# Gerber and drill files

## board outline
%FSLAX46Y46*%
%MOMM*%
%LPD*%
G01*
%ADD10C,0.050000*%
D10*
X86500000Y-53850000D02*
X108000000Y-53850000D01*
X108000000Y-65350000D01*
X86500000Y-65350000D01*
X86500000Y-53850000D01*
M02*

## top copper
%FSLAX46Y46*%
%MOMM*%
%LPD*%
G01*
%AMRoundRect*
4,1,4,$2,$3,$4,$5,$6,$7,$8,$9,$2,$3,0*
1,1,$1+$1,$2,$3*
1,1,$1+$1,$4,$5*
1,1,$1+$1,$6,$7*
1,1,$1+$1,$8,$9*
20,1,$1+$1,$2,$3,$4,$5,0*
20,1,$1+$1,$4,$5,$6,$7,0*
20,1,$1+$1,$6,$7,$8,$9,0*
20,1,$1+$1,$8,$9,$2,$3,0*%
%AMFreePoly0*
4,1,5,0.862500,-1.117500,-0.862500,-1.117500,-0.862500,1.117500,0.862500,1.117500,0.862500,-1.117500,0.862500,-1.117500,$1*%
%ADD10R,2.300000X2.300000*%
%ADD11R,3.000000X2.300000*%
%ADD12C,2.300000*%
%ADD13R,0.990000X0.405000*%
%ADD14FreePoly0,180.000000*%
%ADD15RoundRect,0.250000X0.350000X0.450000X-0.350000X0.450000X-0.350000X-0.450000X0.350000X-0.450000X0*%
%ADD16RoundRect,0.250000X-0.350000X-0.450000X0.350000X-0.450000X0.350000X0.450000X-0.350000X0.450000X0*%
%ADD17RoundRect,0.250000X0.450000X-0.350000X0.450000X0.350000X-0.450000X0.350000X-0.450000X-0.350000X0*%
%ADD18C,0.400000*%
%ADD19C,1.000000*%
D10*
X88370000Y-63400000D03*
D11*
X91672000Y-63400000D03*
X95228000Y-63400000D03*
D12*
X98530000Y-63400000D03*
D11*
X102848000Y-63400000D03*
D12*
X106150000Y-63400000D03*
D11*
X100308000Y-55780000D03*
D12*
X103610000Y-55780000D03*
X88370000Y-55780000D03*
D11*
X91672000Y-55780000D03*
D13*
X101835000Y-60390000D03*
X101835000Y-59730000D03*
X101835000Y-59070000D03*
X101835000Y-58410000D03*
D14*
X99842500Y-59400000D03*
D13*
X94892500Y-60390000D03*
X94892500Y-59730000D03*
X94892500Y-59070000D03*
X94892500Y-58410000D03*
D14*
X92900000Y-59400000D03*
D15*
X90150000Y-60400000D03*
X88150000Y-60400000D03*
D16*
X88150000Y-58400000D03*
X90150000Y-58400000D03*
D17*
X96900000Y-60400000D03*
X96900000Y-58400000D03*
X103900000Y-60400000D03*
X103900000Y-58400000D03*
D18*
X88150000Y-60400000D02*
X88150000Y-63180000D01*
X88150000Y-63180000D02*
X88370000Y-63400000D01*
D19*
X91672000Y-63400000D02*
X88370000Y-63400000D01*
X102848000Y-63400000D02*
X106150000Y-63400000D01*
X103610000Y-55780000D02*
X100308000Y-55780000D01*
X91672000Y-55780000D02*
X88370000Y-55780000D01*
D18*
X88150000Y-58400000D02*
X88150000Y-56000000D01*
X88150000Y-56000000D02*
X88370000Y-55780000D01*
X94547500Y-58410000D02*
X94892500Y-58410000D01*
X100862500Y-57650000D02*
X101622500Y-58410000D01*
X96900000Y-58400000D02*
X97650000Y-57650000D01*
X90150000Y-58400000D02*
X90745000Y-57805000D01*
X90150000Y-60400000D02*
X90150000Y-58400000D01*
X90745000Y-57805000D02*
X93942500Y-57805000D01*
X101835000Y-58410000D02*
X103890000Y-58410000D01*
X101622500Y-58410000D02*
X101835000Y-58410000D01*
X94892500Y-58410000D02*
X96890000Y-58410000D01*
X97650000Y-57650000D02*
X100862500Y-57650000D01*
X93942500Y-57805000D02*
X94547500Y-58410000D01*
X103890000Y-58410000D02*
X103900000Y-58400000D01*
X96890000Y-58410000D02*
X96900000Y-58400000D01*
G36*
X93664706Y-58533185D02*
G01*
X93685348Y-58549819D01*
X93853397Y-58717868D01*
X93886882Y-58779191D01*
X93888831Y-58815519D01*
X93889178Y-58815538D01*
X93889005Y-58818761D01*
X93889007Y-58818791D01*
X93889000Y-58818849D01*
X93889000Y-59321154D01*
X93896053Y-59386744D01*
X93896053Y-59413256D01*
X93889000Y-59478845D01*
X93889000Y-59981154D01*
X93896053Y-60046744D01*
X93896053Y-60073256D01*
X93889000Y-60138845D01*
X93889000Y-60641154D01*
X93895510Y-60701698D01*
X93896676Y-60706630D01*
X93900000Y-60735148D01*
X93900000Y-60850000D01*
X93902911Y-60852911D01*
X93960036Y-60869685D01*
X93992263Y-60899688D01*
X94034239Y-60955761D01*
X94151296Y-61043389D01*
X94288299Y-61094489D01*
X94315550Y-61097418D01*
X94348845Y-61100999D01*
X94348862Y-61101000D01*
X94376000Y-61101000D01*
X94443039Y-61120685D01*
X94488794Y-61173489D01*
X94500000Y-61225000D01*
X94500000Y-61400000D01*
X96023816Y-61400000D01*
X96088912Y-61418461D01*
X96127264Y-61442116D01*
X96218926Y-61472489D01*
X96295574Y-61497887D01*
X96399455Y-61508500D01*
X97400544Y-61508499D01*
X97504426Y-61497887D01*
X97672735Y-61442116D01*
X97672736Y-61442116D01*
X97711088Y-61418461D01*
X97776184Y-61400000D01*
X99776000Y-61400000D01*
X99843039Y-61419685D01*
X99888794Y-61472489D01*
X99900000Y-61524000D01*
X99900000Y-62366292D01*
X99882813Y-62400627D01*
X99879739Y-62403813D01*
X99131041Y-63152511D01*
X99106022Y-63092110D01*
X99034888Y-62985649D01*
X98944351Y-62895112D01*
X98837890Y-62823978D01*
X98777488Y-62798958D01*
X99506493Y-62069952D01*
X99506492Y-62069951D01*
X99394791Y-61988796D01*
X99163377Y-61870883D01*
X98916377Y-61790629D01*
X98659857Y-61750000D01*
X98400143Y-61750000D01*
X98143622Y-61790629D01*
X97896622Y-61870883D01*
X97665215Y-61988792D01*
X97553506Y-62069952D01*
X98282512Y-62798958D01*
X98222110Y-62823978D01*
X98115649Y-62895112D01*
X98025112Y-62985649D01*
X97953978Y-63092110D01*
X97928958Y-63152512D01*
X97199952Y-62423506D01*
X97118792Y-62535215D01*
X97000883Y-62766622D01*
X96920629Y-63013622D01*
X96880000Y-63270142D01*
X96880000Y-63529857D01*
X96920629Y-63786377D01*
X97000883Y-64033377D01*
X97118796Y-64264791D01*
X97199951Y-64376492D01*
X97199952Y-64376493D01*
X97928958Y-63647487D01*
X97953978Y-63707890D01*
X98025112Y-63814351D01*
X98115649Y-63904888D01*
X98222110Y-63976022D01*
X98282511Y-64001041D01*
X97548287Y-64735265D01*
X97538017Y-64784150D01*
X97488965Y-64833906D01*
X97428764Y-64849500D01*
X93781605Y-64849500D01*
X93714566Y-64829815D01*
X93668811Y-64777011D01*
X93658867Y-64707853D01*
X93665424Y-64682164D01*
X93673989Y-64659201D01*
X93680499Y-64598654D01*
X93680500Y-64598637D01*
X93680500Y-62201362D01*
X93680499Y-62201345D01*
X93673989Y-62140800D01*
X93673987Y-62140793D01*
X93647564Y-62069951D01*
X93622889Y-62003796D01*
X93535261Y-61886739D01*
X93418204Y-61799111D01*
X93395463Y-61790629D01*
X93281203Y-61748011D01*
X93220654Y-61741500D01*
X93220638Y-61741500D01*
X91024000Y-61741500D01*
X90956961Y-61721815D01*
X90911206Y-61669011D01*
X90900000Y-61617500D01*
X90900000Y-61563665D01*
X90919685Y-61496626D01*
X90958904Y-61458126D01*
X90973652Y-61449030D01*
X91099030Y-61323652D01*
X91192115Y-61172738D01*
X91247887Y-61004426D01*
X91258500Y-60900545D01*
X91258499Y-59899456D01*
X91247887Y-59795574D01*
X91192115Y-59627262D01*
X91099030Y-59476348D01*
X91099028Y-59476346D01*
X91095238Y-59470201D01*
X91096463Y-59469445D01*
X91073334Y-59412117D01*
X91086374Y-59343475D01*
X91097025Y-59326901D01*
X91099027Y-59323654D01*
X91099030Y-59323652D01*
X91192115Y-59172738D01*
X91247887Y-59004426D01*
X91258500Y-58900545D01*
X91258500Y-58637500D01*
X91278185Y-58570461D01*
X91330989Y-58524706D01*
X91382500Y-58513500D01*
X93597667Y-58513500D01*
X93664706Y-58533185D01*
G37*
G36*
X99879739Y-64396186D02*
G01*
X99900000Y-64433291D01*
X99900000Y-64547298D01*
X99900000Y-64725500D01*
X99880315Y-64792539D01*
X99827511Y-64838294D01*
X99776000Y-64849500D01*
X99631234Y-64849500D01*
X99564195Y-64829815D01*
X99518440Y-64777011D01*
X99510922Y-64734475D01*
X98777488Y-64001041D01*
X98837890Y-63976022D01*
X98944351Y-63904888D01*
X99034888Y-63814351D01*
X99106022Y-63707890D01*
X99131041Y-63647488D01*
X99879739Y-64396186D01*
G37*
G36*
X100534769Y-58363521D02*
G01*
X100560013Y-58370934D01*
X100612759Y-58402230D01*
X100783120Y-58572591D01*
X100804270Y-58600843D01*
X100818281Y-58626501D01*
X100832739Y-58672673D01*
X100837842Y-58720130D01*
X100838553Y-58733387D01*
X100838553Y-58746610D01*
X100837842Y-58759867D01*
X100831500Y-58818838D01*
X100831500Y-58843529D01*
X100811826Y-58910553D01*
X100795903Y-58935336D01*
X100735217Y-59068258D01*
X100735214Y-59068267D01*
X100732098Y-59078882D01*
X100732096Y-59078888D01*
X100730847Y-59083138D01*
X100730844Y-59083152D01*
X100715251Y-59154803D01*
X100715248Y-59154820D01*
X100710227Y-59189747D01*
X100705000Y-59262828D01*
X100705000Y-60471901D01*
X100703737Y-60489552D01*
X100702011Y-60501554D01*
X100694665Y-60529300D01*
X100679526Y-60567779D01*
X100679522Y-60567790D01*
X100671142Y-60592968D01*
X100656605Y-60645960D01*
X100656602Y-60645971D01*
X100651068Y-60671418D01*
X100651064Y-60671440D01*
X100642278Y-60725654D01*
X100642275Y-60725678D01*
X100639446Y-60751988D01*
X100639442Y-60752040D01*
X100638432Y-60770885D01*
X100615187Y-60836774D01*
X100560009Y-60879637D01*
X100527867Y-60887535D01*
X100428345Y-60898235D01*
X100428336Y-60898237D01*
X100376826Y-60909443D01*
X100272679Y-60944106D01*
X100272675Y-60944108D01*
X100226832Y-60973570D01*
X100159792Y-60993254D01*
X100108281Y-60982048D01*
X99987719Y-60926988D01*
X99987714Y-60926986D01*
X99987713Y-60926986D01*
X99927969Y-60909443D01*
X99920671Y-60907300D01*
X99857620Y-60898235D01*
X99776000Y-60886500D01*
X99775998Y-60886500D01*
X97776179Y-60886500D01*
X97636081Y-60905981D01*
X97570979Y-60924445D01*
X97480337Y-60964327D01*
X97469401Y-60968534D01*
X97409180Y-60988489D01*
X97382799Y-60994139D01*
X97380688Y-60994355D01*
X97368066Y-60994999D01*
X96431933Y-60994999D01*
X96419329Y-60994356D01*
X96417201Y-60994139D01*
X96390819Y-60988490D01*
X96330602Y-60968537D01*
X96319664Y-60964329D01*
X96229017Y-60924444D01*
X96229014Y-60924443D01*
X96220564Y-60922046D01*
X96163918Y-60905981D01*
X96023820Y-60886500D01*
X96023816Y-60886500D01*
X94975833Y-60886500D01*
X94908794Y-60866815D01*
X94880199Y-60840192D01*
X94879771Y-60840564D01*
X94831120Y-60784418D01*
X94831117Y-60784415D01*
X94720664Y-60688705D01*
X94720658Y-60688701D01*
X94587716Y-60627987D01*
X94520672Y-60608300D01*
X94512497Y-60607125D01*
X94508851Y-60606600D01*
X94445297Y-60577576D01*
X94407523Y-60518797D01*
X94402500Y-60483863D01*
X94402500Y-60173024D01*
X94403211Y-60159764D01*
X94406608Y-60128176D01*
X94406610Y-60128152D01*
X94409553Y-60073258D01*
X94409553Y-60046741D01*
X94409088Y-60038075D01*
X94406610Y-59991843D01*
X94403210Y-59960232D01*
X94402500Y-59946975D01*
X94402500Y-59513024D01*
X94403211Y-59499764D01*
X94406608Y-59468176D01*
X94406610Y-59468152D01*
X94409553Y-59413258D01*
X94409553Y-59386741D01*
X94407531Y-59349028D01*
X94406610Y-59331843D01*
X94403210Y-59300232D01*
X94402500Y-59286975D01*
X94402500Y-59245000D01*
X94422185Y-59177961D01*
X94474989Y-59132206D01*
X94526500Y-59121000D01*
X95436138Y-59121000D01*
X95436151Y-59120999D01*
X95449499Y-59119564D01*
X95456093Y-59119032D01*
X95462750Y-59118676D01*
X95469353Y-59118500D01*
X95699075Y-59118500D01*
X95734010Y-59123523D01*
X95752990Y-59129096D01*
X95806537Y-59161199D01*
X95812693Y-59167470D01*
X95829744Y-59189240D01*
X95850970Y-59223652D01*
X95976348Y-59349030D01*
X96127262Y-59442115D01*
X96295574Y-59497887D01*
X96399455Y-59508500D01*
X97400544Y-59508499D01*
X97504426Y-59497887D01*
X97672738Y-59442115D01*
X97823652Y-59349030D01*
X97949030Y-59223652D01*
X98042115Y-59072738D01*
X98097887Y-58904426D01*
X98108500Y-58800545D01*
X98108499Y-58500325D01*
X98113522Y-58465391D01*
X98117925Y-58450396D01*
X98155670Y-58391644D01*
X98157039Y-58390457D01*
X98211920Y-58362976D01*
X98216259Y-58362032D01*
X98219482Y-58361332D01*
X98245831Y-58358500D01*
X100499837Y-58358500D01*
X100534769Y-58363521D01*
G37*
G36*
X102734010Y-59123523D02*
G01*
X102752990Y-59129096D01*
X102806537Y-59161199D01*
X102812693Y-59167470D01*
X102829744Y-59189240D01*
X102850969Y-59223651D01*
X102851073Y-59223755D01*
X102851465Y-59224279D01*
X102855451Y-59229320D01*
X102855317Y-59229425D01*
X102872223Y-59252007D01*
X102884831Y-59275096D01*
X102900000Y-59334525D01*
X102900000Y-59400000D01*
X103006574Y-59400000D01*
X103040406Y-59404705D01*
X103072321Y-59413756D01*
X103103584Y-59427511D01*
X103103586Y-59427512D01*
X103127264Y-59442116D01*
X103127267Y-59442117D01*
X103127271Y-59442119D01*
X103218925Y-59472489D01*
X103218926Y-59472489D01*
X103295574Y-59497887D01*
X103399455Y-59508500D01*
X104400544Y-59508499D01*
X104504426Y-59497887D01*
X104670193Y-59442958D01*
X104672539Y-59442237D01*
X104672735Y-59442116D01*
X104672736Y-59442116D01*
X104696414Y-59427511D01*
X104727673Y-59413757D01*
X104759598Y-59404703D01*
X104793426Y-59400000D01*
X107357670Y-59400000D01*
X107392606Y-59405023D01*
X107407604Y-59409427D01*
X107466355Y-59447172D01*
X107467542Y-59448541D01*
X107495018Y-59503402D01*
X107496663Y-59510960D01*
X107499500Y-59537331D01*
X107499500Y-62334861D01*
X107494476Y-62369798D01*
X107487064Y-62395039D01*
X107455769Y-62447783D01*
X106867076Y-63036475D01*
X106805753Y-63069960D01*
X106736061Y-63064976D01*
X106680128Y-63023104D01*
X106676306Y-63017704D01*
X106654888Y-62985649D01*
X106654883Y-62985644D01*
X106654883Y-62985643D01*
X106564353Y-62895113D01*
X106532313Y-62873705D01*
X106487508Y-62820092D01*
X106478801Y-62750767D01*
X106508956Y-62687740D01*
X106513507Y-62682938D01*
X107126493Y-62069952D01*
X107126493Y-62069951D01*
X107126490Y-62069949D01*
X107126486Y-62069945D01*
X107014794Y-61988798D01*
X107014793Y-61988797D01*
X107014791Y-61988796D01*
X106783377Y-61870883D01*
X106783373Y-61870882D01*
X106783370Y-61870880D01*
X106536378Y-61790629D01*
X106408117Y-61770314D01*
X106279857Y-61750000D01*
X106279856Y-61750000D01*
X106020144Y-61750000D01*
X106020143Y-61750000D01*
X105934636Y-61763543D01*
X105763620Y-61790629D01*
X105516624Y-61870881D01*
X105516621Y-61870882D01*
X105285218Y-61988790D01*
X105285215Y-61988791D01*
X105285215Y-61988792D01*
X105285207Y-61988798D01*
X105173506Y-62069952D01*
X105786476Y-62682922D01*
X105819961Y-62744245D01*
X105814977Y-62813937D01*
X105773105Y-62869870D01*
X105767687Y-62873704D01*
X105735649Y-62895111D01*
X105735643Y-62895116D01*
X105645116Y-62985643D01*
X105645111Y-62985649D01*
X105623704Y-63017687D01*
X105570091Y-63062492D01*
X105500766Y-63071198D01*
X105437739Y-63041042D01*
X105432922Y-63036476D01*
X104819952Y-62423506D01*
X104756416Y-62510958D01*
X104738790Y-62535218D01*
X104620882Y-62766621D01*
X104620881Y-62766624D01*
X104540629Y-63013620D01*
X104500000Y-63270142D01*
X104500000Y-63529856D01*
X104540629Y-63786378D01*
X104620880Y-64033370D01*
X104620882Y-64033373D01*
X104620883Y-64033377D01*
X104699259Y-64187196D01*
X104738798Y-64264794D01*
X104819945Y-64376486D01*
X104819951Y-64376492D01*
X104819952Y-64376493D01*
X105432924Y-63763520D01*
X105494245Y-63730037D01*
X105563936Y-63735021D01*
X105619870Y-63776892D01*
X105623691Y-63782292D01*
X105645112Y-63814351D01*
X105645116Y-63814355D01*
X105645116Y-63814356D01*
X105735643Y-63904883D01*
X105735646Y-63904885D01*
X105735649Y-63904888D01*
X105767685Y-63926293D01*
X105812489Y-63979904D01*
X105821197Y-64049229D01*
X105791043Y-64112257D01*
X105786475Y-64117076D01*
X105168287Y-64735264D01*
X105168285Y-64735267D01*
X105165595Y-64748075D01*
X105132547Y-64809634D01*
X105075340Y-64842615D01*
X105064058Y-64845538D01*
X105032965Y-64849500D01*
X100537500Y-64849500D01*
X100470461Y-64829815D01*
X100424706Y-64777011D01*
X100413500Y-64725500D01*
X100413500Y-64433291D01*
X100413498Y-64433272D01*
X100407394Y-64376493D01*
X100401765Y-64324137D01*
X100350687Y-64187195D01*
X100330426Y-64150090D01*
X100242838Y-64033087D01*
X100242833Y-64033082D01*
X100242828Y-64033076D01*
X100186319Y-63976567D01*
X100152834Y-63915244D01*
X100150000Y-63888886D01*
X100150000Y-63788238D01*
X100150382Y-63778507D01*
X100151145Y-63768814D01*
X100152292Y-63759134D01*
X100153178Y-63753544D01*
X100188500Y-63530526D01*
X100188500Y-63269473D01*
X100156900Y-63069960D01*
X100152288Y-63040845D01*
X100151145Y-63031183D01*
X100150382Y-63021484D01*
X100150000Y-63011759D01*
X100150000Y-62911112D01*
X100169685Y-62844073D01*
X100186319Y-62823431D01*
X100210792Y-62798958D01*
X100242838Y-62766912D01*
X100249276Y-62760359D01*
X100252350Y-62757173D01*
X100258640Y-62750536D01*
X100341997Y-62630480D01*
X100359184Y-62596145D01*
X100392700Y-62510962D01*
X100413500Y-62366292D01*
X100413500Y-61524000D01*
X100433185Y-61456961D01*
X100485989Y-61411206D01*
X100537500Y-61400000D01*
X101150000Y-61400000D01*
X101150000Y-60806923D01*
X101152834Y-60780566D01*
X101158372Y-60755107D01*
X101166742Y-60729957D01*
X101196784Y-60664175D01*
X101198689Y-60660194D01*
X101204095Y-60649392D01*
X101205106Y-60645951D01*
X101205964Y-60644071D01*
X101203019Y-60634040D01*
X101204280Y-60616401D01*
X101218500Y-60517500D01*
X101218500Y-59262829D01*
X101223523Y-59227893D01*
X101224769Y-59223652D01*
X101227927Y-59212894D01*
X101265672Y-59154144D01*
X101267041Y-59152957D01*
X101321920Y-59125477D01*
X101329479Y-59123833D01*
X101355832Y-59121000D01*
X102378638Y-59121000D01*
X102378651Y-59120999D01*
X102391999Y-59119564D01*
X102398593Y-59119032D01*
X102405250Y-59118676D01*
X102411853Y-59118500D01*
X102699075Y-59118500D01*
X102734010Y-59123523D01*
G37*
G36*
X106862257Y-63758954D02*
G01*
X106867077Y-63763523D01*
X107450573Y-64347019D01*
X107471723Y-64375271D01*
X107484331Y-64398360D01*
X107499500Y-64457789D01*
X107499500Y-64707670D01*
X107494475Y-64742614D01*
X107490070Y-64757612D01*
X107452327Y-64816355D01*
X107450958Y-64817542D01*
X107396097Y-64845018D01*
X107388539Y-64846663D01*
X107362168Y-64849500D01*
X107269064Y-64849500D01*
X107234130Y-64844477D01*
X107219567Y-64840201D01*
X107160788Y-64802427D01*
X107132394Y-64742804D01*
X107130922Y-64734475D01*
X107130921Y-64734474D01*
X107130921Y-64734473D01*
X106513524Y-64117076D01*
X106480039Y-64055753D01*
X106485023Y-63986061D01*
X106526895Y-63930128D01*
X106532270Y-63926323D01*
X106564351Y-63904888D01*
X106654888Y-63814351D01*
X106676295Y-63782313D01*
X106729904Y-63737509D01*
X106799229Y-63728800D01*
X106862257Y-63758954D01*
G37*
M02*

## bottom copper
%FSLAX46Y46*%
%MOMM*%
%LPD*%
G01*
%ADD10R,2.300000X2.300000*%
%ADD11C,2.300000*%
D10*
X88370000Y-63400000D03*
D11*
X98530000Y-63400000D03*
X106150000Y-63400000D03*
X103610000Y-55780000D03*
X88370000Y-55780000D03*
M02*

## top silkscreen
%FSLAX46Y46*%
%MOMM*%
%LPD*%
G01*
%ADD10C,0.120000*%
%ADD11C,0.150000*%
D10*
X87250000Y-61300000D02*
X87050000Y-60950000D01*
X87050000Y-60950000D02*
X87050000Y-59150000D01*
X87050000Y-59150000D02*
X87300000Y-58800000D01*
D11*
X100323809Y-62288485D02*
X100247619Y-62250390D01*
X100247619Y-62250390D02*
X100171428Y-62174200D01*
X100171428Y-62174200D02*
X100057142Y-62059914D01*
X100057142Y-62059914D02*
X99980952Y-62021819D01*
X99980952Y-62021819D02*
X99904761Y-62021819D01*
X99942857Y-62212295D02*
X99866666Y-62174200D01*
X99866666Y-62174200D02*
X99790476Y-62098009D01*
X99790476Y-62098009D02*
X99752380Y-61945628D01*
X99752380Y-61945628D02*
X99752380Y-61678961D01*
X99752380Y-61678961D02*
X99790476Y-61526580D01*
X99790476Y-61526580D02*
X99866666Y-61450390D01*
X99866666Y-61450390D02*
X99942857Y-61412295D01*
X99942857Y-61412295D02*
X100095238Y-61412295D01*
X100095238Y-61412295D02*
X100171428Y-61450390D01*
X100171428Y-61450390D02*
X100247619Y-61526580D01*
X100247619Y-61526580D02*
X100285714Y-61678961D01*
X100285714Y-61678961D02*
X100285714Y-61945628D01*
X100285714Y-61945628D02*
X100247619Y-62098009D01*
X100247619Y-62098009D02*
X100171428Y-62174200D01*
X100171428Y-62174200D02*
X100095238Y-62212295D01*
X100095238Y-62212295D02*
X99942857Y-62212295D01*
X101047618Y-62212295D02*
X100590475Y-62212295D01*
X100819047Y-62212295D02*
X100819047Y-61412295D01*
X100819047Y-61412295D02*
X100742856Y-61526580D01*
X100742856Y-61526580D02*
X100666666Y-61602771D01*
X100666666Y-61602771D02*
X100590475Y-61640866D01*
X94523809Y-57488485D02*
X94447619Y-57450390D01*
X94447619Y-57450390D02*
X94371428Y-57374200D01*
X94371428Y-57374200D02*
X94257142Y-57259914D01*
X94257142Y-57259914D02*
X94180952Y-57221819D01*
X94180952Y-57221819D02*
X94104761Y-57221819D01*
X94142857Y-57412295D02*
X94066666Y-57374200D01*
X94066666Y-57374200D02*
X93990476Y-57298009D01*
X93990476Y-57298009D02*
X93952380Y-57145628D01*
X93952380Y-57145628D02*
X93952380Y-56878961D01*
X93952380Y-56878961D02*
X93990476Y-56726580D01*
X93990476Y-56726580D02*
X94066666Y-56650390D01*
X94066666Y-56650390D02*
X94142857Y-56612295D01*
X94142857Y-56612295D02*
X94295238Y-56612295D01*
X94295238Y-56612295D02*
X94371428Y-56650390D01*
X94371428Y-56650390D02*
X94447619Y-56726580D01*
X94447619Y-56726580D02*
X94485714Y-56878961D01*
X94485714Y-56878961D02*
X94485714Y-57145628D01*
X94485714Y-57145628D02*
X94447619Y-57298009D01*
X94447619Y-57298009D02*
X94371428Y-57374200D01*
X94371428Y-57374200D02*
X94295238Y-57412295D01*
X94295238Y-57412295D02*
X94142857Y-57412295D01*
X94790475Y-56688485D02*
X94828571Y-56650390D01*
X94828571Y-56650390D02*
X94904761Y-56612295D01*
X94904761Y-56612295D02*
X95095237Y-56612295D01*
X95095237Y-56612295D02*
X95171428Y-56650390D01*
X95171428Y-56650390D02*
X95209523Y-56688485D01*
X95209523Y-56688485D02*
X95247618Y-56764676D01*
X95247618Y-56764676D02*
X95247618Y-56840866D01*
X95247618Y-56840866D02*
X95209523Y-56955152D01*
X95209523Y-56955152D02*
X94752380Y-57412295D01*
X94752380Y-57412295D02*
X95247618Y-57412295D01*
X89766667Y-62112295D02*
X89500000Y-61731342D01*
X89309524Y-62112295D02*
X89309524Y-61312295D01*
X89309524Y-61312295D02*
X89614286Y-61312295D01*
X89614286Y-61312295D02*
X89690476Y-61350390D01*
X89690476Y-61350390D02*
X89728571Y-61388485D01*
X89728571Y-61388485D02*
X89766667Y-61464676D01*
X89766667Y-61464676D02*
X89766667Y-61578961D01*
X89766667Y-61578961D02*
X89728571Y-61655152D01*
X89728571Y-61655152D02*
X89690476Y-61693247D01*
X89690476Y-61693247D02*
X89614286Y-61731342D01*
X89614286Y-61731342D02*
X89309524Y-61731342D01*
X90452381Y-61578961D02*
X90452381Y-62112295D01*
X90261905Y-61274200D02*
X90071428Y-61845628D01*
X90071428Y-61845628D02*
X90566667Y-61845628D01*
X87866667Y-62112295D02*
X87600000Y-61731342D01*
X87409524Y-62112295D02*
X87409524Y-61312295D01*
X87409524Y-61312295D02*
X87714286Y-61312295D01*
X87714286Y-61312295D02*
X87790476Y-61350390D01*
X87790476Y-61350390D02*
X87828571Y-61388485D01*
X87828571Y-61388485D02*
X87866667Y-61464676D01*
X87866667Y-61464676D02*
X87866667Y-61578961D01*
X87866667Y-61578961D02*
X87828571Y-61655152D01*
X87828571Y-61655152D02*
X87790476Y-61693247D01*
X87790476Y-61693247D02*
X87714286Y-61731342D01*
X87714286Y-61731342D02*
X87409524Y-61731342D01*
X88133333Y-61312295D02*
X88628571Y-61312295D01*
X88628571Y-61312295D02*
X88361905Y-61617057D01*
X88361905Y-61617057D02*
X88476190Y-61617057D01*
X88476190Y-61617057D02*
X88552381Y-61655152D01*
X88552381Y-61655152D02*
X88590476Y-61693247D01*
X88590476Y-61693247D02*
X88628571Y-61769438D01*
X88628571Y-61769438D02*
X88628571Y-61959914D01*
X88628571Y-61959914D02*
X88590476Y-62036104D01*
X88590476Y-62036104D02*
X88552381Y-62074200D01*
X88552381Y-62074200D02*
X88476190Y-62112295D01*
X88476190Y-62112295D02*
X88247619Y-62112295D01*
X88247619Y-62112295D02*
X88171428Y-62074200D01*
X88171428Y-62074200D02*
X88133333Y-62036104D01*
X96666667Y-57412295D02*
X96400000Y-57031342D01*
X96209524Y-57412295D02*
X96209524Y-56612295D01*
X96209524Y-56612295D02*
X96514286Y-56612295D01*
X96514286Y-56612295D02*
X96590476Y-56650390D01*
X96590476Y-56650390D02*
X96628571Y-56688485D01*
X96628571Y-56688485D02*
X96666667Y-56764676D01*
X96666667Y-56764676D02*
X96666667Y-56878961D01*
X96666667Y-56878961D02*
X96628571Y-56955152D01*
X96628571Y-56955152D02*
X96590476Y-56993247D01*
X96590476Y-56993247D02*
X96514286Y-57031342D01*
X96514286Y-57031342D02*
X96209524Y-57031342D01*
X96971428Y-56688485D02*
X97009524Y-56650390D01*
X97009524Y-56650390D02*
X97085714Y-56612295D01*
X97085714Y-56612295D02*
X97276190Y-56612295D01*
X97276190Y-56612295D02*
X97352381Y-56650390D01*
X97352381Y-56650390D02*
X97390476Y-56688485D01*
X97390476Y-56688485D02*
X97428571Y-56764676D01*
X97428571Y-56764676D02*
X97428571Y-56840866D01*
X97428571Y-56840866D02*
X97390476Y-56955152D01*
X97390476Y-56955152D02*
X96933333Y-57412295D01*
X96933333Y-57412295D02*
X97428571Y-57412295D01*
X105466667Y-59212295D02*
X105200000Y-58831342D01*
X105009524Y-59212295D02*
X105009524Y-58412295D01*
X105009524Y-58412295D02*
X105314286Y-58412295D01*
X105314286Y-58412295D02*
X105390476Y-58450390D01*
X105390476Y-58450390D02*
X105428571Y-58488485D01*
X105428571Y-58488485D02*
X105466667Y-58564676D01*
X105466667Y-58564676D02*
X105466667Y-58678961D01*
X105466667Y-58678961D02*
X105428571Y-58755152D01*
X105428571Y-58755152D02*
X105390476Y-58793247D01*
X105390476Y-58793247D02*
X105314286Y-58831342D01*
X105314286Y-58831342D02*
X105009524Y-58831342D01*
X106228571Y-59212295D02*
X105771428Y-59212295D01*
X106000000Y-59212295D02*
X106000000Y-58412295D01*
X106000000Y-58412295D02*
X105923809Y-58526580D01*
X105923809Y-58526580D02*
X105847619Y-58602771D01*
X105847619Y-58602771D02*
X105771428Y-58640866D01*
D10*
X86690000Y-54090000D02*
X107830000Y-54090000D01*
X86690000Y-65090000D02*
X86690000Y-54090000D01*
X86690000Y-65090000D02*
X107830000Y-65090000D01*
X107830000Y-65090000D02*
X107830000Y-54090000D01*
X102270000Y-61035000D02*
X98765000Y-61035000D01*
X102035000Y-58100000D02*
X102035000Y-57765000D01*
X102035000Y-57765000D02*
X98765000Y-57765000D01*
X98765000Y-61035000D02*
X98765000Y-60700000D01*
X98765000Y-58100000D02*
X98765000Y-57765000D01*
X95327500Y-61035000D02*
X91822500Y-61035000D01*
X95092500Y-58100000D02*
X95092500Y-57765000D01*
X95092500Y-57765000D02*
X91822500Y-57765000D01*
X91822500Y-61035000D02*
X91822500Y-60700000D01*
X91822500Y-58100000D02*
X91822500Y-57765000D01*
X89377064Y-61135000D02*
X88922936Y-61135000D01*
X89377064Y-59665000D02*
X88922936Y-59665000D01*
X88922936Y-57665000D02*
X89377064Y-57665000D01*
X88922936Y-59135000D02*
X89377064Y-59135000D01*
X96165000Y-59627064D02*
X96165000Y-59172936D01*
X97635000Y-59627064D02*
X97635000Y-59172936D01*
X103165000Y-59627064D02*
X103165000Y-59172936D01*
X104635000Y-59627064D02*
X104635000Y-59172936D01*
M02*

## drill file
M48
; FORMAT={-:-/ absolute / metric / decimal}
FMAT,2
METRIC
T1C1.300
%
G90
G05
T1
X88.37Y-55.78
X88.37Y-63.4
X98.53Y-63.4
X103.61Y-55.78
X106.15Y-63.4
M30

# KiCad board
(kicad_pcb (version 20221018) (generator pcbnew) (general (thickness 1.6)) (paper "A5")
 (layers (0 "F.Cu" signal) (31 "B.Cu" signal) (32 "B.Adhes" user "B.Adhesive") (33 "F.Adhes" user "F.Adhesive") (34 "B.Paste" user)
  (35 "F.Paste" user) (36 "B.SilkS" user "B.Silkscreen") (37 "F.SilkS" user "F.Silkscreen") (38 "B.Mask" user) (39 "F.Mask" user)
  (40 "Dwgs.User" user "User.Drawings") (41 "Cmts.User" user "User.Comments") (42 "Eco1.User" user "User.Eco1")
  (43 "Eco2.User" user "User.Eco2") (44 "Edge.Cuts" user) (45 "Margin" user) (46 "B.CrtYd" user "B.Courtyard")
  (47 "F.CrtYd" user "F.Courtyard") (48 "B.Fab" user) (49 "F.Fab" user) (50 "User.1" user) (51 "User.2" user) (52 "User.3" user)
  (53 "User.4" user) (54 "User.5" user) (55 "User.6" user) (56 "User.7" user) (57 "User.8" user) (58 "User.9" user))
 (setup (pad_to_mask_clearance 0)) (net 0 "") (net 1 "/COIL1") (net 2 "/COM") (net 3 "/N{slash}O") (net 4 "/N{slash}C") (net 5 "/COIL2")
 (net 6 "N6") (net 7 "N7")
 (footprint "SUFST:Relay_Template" (layer "F.Cu") (at 88.37 63.4)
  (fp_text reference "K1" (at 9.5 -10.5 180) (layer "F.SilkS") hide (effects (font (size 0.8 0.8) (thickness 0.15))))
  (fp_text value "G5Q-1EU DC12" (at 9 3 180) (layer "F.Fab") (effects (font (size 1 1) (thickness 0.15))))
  (fp_line (start -1.68 -9.31) (end 19.46 -9.31) (stroke (width 0.12) (type solid)) (layer "F.SilkS"))
  (fp_line (start -1.68 1.69) (end -1.68 -9.31) (stroke (width 0.12) (type solid)) (layer "F.SilkS"))
  (fp_line (start -1.68 1.69) (end 19.46 1.69) (stroke (width 0.12) (type solid)) (layer "F.SilkS"))
  (fp_line (start 19.46 1.69) (end 19.46 -9.31) (stroke (width 0.12) (type solid)) (layer "F.SilkS"))
  (pad "1" thru_hole rect (at 0 0 180) (size 2.3 2.3) (drill 1.3) (layers "*.Cu" "*.Mask") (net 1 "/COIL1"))
  (pad "1" smd rect (at 3.302 0 270) (size 2.3 3) (layers "F.Cu" "F.Paste" "F.Mask") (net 1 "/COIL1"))
  (pad "2" smd rect (at 6.858 0 270) (size 2.3 3) (layers "F.Cu" "F.Paste" "F.Mask") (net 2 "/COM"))
  (pad "2" thru_hole circle (at 10.16 0 180) (size 2.3 2.3) (drill 1.3) (layers "*.Cu" "*.Mask") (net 2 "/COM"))
  (pad "3" smd rect (at 14.478 0 270) (size 2.3 3) (layers "F.Cu" "F.Paste" "F.Mask") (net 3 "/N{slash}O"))
  (pad "3" thru_hole circle (at 17.78 0 180) (size 2.3 2.3) (drill 1.3) (layers "*.Cu" "*.Mask") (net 3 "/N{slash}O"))
  (pad "4" smd rect (at 11.938 -7.62 270) (size 2.3 3) (layers "F.Cu" "F.Paste" "F.Mask") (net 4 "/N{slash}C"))
  (pad "4" thru_hole circle (at 15.24 -7.62 180) (size 2.3 2.3) (drill 1.3) (layers "*.Cu" "*.Mask") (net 4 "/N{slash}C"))
  (pad "5" thru_hole circle (at 0 -7.62 180) (size 2.3 2.3) (drill 1.3) (layers "*.Cu" "*.Mask") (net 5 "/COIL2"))
  (pad "5" smd rect (at 3.302 -7.62 270) (size 2.3 3) (layers "F.Cu" "F.Paste" "F.Mask") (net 5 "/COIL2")))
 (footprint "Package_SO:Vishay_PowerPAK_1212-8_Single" (layer "F.Cu") (at 100.4 59.4 180)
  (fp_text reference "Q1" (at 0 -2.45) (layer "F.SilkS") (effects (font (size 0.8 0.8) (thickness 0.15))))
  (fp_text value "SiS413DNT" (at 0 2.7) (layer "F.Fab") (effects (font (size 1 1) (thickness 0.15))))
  (fp_line (start -1.87 -1.635) (end 1.635 -1.635) (stroke (width 0.12) (type solid)) (layer "F.SilkS"))
  (fp_line (start -1.635 1.3) (end -1.635 1.635) (stroke (width 0.12) (type solid)) (layer "F.SilkS"))
  (fp_line (start -1.635 1.635) (end 1.635 1.635) (stroke (width 0.12) (type solid)) (layer "F.SilkS"))
  (fp_line (start 1.635 -1.635) (end 1.635 -1.3) (stroke (width 0.12) (type solid)) (layer "F.SilkS"))
  (fp_line (start 1.635 1.3) (end 1.635 1.635) (stroke (width 0.12) (type solid)) (layer "F.SilkS"))
  (pad "1" smd rect (at -1.435 -0.99 180) (size 0.99 0.405) (layers "F.Cu" "F.Paste" "F.Mask") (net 3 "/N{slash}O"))
  (pad "2" smd rect (at -1.435 -0.33 180) (size 0.99 0.405) (layers "F.Cu" "F.Paste" "F.Mask") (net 3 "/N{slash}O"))
  (pad "3" smd rect (at -1.435 0.33 180) (size 0.99 0.405) (layers "F.Cu" "F.Paste" "F.Mask") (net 3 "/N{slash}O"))
  (pad "4" smd rect (at -1.435 0.99 180) (size 0.99 0.405) (layers "F.Cu" "F.Paste" "F.Mask") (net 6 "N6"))
  (pad "5" smd custom (at 0.5575 0 180) (size 1.725 2.235) (layers "F.Cu" "F.Paste" "F.Mask") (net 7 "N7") (zone_connect 2)
   (options (clearance outline) (anchor rect)) (primitives)))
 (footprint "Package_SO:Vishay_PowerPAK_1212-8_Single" (layer "F.Cu") (at 93.4575 59.4 180)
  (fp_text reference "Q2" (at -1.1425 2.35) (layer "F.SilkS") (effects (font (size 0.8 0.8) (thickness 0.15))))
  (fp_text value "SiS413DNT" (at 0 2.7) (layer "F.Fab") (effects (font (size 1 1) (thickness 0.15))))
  (fp_line (start -1.87 -1.635) (end 1.635 -1.635) (stroke (width 0.12) (type solid)) (layer "F.SilkS"))
  (fp_line (start -1.635 1.3) (end -1.635 1.635) (stroke (width 0.12) (type solid)) (layer "F.SilkS"))
  (fp_line (start -1.635 1.635) (end 1.635 1.635) (stroke (width 0.12) (type solid)) (layer "F.SilkS"))
  (fp_line (start 1.635 -1.635) (end 1.635 -1.3) (stroke (width 0.12) (type solid)) (layer "F.SilkS"))
  (fp_line (start 1.635 1.3) (end 1.635 1.635) (stroke (width 0.12) (type solid)) (layer "F.SilkS"))
  (pad "1" smd rect (at -1.435 -0.99 180) (size 0.99 0.405) (layers "F.Cu" "F.Paste" "F.Mask") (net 7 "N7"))
  (pad "2" smd rect (at -1.435 -0.33 180) (size 0.99 0.405) (layers "F.Cu" "F.Paste" "F.Mask") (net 7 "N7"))
  (pad "3" smd rect (at -1.435 0.33 180) (size 0.99 0.405) (layers "F.Cu" "F.Paste" "F.Mask") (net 7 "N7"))
  (pad "4" smd rect (at -1.435 0.99 180) (size 0.99 0.405) (layers "F.Cu" "F.Paste" "F.Mask") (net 6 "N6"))
  (pad "5" smd custom (at 0.5575 0 180) (size 1.725 2.235) (layers "F.Cu" "F.Paste" "F.Mask") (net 2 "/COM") (zone_connect 2)
   (options (clearance outline) (anchor rect)) (primitives)))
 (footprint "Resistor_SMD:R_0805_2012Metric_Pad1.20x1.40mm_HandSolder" (layer "F.Cu") (at 89.15 60.4 180)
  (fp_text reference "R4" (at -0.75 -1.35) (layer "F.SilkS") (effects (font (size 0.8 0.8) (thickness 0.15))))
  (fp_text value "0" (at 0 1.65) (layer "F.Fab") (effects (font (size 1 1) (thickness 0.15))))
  (fp_line (start -0.227064 -0.735) (end 0.227064 -0.735) (stroke (width 0.12) (type solid)) (layer "F.SilkS"))
  (fp_line (start -0.227064 0.735) (end 0.227064 0.735) (stroke (width 0.12) (type solid)) (layer "F.SilkS"))
  (pad "1" smd roundrect (at -1 0 180) (size 1.2 1.4) (layers "F.Cu" "F.Paste" "F.Mask") (roundrect_rratio 0.2083333333) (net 6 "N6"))
  (pad "2" smd roundrect (at 1 0 180) (size 1.2 1.4) (layers "F.Cu" "F.Paste" "F.Mask") (roundrect_rratio 0.2083333333) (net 1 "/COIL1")))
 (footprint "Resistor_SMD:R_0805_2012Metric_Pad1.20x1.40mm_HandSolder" (layer "F.Cu") (at 89.15 58.4)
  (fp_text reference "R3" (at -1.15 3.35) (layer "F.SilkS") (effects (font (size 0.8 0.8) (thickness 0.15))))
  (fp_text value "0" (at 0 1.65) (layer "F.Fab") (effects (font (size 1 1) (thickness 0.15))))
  (fp_line (start -0.227064 -0.735) (end 0.227064 -0.735) (stroke (width 0.12) (type solid)) (layer "F.SilkS"))
  (fp_line (start -0.227064 0.735) (end 0.227064 0.735) (stroke (width 0.12) (type solid)) (layer "F.SilkS"))
  (pad "1" smd roundrect (at -1 0) (size 1.2 1.4) (layers "F.Cu" "F.Paste" "F.Mask") (roundrect_rratio 0.2083333333) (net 5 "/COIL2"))
  (pad "2" smd roundrect (at 1 0) (size 1.2 1.4) (layers "F.Cu" "F.Paste" "F.Mask") (roundrect_rratio 0.2083333333) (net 6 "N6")))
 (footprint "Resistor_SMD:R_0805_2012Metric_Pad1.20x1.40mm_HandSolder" (layer "F.Cu") (at 96.9 59.4 90)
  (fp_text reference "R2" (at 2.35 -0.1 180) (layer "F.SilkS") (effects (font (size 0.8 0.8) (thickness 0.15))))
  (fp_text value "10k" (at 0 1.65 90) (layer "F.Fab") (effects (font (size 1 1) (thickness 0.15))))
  (fp_line (start -0.227064 -0.735) (end 0.227064 -0.735) (stroke (width 0.12) (type solid)) (layer "F.SilkS"))
  (fp_line (start -0.227064 0.735) (end 0.227064 0.735) (stroke (width 0.12) (type solid)) (layer "F.SilkS"))
  (pad "1" smd roundrect (at -1 0 90) (size 1.2 1.4) (layers "F.Cu" "F.Paste" "F.Mask") (roundrect_rratio 0.2083333333) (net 7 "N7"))
  (pad "2" smd roundrect (at 1 0 90) (size 1.2 1.4) (layers "F.Cu" "F.Paste" "F.Mask") (roundrect_rratio 0.2083333333) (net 6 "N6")))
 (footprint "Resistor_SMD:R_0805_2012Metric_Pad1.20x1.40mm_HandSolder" (layer "F.Cu") (at 103.9 59.4 90)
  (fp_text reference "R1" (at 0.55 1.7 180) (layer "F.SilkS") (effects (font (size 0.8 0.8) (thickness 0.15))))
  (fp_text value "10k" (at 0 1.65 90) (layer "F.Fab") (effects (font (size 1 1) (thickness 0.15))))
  (fp_line (start -0.227064 -0.735) (end 0.227064 -0.735) (stroke (width 0.12) (type solid)) (layer "F.SilkS"))
  (fp_line (start -0.227064 0.735) (end 0.227064 0.735) (stroke (width 0.12) (type solid)) (layer "F.SilkS"))
  (pad "1" smd roundrect (at -1 0 90) (size 1.2 1.4) (layers "F.Cu" "F.Paste" "F.Mask") (roundrect_rratio 0.2083333333) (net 3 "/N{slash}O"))
  (pad "2" smd roundrect (at 1 0 90) (size 1.2 1.4) (layers "F.Cu" "F.Paste" "F.Mask") (roundrect_rratio 0.2083333333) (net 6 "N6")))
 (gr_line (start 87.25 61.3) (end 87.05 60.95) (stroke (width 0.12) (type default)) (layer "F.SilkS"))
 (gr_line (start 87.05 60.95) (end 87.05 59.15) (stroke (width 0.12) (type default)) (layer "F.SilkS"))
 (gr_line (start 87.05 59.15) (end 87.3 58.8) (stroke (width 0.12) (type default)) (layer "F.SilkS"))
 (gr_rect (start 86.5 53.85) (end 108 65.35) (stroke (width 0.05) (type default)) (fill none) (layer "Edge.Cuts"))
 (segment (start 88.15 60.4) (end 88.15 63.18) (width 0.4) (layer "F.Cu") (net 1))
 (segment (start 88.15 63.18) (end 88.37 63.4) (width 0.4) (layer "F.Cu") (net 1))
 (segment (start 91.672 63.4) (end 88.37 63.4) (width 1) (layer "F.Cu") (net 1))
 (segment (start 102.848 63.4) (end 106.15 63.4) (width 1) (layer "F.Cu") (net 3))
 (segment (start 103.61 55.78) (end 100.308 55.78) (width 1) (layer "F.Cu") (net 4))
 (segment (start 91.672 55.78) (end 88.37 55.78) (width 1) (layer "F.Cu") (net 5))
 (segment (start 88.15 58.4) (end 88.15 56) (width 0.4) (layer "F.Cu") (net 5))
 (segment (start 88.15 56) (end 88.37 55.78) (width 0.4) (layer "F.Cu") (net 5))
 (segment (start 94.5475 58.41) (end 94.8925 58.41) (width 0.4) (layer "F.Cu") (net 6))
 (segment (start 100.8625 57.65) (end 101.6225 58.41) (width 0.4) (layer "F.Cu") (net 6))
 (segment (start 96.9 58.4) (end 97.65 57.65) (width 0.4) (layer "F.Cu") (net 6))
 (segment (start 90.15 58.4) (end 90.745 57.805) (width 0.4) (layer "F.Cu") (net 6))
 (segment (start 90.15 60.4) (end 90.15 58.4) (width 0.4) (layer "F.Cu") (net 6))
 (segment (start 90.745 57.805) (end 93.9425 57.805) (width 0.4) (layer "F.Cu") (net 6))
 (segment (start 101.835 58.41) (end 103.89 58.41) (width 0.4) (layer "F.Cu") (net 6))
 (segment (start 101.6225 58.41) (end 101.835 58.41) (width 0.4) (layer "F.Cu") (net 6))
 (segment (start 94.8925 58.41) (end 96.89 58.41) (width 0.4) (layer "F.Cu") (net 6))
 (segment (start 97.65 57.65) (end 100.8625 57.65) (width 0.4) (layer "F.Cu") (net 6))
 (segment (start 93.9425 57.805) (end 94.5475 58.41) (width 0.4) (layer "F.Cu") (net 6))
 (segment (start 103.89 58.41) (end 103.9 58.4) (width 0.4) (layer "F.Cu") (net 6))
 (segment (start 96.89 58.41) (end 96.9 58.4) (width 0.4) (layer "F.Cu") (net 6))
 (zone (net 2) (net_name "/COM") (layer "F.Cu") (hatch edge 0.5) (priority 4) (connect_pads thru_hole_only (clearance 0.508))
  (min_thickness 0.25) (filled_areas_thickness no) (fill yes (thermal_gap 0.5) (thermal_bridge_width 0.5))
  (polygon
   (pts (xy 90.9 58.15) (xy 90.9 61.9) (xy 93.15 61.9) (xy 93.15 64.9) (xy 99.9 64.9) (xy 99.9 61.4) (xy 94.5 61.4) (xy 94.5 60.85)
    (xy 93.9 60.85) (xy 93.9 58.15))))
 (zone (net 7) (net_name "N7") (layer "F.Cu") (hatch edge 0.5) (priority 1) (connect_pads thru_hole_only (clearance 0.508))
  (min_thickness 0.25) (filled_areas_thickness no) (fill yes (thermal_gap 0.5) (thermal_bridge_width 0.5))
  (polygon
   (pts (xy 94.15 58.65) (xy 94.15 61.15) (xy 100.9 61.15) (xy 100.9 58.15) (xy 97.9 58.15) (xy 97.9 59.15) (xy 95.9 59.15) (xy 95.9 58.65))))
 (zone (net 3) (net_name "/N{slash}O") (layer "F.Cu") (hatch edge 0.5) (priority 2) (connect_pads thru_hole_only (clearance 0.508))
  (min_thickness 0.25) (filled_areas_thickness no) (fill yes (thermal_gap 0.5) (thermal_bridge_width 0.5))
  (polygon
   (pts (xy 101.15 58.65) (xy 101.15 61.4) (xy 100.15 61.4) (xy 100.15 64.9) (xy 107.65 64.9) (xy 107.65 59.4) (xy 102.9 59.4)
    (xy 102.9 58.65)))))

